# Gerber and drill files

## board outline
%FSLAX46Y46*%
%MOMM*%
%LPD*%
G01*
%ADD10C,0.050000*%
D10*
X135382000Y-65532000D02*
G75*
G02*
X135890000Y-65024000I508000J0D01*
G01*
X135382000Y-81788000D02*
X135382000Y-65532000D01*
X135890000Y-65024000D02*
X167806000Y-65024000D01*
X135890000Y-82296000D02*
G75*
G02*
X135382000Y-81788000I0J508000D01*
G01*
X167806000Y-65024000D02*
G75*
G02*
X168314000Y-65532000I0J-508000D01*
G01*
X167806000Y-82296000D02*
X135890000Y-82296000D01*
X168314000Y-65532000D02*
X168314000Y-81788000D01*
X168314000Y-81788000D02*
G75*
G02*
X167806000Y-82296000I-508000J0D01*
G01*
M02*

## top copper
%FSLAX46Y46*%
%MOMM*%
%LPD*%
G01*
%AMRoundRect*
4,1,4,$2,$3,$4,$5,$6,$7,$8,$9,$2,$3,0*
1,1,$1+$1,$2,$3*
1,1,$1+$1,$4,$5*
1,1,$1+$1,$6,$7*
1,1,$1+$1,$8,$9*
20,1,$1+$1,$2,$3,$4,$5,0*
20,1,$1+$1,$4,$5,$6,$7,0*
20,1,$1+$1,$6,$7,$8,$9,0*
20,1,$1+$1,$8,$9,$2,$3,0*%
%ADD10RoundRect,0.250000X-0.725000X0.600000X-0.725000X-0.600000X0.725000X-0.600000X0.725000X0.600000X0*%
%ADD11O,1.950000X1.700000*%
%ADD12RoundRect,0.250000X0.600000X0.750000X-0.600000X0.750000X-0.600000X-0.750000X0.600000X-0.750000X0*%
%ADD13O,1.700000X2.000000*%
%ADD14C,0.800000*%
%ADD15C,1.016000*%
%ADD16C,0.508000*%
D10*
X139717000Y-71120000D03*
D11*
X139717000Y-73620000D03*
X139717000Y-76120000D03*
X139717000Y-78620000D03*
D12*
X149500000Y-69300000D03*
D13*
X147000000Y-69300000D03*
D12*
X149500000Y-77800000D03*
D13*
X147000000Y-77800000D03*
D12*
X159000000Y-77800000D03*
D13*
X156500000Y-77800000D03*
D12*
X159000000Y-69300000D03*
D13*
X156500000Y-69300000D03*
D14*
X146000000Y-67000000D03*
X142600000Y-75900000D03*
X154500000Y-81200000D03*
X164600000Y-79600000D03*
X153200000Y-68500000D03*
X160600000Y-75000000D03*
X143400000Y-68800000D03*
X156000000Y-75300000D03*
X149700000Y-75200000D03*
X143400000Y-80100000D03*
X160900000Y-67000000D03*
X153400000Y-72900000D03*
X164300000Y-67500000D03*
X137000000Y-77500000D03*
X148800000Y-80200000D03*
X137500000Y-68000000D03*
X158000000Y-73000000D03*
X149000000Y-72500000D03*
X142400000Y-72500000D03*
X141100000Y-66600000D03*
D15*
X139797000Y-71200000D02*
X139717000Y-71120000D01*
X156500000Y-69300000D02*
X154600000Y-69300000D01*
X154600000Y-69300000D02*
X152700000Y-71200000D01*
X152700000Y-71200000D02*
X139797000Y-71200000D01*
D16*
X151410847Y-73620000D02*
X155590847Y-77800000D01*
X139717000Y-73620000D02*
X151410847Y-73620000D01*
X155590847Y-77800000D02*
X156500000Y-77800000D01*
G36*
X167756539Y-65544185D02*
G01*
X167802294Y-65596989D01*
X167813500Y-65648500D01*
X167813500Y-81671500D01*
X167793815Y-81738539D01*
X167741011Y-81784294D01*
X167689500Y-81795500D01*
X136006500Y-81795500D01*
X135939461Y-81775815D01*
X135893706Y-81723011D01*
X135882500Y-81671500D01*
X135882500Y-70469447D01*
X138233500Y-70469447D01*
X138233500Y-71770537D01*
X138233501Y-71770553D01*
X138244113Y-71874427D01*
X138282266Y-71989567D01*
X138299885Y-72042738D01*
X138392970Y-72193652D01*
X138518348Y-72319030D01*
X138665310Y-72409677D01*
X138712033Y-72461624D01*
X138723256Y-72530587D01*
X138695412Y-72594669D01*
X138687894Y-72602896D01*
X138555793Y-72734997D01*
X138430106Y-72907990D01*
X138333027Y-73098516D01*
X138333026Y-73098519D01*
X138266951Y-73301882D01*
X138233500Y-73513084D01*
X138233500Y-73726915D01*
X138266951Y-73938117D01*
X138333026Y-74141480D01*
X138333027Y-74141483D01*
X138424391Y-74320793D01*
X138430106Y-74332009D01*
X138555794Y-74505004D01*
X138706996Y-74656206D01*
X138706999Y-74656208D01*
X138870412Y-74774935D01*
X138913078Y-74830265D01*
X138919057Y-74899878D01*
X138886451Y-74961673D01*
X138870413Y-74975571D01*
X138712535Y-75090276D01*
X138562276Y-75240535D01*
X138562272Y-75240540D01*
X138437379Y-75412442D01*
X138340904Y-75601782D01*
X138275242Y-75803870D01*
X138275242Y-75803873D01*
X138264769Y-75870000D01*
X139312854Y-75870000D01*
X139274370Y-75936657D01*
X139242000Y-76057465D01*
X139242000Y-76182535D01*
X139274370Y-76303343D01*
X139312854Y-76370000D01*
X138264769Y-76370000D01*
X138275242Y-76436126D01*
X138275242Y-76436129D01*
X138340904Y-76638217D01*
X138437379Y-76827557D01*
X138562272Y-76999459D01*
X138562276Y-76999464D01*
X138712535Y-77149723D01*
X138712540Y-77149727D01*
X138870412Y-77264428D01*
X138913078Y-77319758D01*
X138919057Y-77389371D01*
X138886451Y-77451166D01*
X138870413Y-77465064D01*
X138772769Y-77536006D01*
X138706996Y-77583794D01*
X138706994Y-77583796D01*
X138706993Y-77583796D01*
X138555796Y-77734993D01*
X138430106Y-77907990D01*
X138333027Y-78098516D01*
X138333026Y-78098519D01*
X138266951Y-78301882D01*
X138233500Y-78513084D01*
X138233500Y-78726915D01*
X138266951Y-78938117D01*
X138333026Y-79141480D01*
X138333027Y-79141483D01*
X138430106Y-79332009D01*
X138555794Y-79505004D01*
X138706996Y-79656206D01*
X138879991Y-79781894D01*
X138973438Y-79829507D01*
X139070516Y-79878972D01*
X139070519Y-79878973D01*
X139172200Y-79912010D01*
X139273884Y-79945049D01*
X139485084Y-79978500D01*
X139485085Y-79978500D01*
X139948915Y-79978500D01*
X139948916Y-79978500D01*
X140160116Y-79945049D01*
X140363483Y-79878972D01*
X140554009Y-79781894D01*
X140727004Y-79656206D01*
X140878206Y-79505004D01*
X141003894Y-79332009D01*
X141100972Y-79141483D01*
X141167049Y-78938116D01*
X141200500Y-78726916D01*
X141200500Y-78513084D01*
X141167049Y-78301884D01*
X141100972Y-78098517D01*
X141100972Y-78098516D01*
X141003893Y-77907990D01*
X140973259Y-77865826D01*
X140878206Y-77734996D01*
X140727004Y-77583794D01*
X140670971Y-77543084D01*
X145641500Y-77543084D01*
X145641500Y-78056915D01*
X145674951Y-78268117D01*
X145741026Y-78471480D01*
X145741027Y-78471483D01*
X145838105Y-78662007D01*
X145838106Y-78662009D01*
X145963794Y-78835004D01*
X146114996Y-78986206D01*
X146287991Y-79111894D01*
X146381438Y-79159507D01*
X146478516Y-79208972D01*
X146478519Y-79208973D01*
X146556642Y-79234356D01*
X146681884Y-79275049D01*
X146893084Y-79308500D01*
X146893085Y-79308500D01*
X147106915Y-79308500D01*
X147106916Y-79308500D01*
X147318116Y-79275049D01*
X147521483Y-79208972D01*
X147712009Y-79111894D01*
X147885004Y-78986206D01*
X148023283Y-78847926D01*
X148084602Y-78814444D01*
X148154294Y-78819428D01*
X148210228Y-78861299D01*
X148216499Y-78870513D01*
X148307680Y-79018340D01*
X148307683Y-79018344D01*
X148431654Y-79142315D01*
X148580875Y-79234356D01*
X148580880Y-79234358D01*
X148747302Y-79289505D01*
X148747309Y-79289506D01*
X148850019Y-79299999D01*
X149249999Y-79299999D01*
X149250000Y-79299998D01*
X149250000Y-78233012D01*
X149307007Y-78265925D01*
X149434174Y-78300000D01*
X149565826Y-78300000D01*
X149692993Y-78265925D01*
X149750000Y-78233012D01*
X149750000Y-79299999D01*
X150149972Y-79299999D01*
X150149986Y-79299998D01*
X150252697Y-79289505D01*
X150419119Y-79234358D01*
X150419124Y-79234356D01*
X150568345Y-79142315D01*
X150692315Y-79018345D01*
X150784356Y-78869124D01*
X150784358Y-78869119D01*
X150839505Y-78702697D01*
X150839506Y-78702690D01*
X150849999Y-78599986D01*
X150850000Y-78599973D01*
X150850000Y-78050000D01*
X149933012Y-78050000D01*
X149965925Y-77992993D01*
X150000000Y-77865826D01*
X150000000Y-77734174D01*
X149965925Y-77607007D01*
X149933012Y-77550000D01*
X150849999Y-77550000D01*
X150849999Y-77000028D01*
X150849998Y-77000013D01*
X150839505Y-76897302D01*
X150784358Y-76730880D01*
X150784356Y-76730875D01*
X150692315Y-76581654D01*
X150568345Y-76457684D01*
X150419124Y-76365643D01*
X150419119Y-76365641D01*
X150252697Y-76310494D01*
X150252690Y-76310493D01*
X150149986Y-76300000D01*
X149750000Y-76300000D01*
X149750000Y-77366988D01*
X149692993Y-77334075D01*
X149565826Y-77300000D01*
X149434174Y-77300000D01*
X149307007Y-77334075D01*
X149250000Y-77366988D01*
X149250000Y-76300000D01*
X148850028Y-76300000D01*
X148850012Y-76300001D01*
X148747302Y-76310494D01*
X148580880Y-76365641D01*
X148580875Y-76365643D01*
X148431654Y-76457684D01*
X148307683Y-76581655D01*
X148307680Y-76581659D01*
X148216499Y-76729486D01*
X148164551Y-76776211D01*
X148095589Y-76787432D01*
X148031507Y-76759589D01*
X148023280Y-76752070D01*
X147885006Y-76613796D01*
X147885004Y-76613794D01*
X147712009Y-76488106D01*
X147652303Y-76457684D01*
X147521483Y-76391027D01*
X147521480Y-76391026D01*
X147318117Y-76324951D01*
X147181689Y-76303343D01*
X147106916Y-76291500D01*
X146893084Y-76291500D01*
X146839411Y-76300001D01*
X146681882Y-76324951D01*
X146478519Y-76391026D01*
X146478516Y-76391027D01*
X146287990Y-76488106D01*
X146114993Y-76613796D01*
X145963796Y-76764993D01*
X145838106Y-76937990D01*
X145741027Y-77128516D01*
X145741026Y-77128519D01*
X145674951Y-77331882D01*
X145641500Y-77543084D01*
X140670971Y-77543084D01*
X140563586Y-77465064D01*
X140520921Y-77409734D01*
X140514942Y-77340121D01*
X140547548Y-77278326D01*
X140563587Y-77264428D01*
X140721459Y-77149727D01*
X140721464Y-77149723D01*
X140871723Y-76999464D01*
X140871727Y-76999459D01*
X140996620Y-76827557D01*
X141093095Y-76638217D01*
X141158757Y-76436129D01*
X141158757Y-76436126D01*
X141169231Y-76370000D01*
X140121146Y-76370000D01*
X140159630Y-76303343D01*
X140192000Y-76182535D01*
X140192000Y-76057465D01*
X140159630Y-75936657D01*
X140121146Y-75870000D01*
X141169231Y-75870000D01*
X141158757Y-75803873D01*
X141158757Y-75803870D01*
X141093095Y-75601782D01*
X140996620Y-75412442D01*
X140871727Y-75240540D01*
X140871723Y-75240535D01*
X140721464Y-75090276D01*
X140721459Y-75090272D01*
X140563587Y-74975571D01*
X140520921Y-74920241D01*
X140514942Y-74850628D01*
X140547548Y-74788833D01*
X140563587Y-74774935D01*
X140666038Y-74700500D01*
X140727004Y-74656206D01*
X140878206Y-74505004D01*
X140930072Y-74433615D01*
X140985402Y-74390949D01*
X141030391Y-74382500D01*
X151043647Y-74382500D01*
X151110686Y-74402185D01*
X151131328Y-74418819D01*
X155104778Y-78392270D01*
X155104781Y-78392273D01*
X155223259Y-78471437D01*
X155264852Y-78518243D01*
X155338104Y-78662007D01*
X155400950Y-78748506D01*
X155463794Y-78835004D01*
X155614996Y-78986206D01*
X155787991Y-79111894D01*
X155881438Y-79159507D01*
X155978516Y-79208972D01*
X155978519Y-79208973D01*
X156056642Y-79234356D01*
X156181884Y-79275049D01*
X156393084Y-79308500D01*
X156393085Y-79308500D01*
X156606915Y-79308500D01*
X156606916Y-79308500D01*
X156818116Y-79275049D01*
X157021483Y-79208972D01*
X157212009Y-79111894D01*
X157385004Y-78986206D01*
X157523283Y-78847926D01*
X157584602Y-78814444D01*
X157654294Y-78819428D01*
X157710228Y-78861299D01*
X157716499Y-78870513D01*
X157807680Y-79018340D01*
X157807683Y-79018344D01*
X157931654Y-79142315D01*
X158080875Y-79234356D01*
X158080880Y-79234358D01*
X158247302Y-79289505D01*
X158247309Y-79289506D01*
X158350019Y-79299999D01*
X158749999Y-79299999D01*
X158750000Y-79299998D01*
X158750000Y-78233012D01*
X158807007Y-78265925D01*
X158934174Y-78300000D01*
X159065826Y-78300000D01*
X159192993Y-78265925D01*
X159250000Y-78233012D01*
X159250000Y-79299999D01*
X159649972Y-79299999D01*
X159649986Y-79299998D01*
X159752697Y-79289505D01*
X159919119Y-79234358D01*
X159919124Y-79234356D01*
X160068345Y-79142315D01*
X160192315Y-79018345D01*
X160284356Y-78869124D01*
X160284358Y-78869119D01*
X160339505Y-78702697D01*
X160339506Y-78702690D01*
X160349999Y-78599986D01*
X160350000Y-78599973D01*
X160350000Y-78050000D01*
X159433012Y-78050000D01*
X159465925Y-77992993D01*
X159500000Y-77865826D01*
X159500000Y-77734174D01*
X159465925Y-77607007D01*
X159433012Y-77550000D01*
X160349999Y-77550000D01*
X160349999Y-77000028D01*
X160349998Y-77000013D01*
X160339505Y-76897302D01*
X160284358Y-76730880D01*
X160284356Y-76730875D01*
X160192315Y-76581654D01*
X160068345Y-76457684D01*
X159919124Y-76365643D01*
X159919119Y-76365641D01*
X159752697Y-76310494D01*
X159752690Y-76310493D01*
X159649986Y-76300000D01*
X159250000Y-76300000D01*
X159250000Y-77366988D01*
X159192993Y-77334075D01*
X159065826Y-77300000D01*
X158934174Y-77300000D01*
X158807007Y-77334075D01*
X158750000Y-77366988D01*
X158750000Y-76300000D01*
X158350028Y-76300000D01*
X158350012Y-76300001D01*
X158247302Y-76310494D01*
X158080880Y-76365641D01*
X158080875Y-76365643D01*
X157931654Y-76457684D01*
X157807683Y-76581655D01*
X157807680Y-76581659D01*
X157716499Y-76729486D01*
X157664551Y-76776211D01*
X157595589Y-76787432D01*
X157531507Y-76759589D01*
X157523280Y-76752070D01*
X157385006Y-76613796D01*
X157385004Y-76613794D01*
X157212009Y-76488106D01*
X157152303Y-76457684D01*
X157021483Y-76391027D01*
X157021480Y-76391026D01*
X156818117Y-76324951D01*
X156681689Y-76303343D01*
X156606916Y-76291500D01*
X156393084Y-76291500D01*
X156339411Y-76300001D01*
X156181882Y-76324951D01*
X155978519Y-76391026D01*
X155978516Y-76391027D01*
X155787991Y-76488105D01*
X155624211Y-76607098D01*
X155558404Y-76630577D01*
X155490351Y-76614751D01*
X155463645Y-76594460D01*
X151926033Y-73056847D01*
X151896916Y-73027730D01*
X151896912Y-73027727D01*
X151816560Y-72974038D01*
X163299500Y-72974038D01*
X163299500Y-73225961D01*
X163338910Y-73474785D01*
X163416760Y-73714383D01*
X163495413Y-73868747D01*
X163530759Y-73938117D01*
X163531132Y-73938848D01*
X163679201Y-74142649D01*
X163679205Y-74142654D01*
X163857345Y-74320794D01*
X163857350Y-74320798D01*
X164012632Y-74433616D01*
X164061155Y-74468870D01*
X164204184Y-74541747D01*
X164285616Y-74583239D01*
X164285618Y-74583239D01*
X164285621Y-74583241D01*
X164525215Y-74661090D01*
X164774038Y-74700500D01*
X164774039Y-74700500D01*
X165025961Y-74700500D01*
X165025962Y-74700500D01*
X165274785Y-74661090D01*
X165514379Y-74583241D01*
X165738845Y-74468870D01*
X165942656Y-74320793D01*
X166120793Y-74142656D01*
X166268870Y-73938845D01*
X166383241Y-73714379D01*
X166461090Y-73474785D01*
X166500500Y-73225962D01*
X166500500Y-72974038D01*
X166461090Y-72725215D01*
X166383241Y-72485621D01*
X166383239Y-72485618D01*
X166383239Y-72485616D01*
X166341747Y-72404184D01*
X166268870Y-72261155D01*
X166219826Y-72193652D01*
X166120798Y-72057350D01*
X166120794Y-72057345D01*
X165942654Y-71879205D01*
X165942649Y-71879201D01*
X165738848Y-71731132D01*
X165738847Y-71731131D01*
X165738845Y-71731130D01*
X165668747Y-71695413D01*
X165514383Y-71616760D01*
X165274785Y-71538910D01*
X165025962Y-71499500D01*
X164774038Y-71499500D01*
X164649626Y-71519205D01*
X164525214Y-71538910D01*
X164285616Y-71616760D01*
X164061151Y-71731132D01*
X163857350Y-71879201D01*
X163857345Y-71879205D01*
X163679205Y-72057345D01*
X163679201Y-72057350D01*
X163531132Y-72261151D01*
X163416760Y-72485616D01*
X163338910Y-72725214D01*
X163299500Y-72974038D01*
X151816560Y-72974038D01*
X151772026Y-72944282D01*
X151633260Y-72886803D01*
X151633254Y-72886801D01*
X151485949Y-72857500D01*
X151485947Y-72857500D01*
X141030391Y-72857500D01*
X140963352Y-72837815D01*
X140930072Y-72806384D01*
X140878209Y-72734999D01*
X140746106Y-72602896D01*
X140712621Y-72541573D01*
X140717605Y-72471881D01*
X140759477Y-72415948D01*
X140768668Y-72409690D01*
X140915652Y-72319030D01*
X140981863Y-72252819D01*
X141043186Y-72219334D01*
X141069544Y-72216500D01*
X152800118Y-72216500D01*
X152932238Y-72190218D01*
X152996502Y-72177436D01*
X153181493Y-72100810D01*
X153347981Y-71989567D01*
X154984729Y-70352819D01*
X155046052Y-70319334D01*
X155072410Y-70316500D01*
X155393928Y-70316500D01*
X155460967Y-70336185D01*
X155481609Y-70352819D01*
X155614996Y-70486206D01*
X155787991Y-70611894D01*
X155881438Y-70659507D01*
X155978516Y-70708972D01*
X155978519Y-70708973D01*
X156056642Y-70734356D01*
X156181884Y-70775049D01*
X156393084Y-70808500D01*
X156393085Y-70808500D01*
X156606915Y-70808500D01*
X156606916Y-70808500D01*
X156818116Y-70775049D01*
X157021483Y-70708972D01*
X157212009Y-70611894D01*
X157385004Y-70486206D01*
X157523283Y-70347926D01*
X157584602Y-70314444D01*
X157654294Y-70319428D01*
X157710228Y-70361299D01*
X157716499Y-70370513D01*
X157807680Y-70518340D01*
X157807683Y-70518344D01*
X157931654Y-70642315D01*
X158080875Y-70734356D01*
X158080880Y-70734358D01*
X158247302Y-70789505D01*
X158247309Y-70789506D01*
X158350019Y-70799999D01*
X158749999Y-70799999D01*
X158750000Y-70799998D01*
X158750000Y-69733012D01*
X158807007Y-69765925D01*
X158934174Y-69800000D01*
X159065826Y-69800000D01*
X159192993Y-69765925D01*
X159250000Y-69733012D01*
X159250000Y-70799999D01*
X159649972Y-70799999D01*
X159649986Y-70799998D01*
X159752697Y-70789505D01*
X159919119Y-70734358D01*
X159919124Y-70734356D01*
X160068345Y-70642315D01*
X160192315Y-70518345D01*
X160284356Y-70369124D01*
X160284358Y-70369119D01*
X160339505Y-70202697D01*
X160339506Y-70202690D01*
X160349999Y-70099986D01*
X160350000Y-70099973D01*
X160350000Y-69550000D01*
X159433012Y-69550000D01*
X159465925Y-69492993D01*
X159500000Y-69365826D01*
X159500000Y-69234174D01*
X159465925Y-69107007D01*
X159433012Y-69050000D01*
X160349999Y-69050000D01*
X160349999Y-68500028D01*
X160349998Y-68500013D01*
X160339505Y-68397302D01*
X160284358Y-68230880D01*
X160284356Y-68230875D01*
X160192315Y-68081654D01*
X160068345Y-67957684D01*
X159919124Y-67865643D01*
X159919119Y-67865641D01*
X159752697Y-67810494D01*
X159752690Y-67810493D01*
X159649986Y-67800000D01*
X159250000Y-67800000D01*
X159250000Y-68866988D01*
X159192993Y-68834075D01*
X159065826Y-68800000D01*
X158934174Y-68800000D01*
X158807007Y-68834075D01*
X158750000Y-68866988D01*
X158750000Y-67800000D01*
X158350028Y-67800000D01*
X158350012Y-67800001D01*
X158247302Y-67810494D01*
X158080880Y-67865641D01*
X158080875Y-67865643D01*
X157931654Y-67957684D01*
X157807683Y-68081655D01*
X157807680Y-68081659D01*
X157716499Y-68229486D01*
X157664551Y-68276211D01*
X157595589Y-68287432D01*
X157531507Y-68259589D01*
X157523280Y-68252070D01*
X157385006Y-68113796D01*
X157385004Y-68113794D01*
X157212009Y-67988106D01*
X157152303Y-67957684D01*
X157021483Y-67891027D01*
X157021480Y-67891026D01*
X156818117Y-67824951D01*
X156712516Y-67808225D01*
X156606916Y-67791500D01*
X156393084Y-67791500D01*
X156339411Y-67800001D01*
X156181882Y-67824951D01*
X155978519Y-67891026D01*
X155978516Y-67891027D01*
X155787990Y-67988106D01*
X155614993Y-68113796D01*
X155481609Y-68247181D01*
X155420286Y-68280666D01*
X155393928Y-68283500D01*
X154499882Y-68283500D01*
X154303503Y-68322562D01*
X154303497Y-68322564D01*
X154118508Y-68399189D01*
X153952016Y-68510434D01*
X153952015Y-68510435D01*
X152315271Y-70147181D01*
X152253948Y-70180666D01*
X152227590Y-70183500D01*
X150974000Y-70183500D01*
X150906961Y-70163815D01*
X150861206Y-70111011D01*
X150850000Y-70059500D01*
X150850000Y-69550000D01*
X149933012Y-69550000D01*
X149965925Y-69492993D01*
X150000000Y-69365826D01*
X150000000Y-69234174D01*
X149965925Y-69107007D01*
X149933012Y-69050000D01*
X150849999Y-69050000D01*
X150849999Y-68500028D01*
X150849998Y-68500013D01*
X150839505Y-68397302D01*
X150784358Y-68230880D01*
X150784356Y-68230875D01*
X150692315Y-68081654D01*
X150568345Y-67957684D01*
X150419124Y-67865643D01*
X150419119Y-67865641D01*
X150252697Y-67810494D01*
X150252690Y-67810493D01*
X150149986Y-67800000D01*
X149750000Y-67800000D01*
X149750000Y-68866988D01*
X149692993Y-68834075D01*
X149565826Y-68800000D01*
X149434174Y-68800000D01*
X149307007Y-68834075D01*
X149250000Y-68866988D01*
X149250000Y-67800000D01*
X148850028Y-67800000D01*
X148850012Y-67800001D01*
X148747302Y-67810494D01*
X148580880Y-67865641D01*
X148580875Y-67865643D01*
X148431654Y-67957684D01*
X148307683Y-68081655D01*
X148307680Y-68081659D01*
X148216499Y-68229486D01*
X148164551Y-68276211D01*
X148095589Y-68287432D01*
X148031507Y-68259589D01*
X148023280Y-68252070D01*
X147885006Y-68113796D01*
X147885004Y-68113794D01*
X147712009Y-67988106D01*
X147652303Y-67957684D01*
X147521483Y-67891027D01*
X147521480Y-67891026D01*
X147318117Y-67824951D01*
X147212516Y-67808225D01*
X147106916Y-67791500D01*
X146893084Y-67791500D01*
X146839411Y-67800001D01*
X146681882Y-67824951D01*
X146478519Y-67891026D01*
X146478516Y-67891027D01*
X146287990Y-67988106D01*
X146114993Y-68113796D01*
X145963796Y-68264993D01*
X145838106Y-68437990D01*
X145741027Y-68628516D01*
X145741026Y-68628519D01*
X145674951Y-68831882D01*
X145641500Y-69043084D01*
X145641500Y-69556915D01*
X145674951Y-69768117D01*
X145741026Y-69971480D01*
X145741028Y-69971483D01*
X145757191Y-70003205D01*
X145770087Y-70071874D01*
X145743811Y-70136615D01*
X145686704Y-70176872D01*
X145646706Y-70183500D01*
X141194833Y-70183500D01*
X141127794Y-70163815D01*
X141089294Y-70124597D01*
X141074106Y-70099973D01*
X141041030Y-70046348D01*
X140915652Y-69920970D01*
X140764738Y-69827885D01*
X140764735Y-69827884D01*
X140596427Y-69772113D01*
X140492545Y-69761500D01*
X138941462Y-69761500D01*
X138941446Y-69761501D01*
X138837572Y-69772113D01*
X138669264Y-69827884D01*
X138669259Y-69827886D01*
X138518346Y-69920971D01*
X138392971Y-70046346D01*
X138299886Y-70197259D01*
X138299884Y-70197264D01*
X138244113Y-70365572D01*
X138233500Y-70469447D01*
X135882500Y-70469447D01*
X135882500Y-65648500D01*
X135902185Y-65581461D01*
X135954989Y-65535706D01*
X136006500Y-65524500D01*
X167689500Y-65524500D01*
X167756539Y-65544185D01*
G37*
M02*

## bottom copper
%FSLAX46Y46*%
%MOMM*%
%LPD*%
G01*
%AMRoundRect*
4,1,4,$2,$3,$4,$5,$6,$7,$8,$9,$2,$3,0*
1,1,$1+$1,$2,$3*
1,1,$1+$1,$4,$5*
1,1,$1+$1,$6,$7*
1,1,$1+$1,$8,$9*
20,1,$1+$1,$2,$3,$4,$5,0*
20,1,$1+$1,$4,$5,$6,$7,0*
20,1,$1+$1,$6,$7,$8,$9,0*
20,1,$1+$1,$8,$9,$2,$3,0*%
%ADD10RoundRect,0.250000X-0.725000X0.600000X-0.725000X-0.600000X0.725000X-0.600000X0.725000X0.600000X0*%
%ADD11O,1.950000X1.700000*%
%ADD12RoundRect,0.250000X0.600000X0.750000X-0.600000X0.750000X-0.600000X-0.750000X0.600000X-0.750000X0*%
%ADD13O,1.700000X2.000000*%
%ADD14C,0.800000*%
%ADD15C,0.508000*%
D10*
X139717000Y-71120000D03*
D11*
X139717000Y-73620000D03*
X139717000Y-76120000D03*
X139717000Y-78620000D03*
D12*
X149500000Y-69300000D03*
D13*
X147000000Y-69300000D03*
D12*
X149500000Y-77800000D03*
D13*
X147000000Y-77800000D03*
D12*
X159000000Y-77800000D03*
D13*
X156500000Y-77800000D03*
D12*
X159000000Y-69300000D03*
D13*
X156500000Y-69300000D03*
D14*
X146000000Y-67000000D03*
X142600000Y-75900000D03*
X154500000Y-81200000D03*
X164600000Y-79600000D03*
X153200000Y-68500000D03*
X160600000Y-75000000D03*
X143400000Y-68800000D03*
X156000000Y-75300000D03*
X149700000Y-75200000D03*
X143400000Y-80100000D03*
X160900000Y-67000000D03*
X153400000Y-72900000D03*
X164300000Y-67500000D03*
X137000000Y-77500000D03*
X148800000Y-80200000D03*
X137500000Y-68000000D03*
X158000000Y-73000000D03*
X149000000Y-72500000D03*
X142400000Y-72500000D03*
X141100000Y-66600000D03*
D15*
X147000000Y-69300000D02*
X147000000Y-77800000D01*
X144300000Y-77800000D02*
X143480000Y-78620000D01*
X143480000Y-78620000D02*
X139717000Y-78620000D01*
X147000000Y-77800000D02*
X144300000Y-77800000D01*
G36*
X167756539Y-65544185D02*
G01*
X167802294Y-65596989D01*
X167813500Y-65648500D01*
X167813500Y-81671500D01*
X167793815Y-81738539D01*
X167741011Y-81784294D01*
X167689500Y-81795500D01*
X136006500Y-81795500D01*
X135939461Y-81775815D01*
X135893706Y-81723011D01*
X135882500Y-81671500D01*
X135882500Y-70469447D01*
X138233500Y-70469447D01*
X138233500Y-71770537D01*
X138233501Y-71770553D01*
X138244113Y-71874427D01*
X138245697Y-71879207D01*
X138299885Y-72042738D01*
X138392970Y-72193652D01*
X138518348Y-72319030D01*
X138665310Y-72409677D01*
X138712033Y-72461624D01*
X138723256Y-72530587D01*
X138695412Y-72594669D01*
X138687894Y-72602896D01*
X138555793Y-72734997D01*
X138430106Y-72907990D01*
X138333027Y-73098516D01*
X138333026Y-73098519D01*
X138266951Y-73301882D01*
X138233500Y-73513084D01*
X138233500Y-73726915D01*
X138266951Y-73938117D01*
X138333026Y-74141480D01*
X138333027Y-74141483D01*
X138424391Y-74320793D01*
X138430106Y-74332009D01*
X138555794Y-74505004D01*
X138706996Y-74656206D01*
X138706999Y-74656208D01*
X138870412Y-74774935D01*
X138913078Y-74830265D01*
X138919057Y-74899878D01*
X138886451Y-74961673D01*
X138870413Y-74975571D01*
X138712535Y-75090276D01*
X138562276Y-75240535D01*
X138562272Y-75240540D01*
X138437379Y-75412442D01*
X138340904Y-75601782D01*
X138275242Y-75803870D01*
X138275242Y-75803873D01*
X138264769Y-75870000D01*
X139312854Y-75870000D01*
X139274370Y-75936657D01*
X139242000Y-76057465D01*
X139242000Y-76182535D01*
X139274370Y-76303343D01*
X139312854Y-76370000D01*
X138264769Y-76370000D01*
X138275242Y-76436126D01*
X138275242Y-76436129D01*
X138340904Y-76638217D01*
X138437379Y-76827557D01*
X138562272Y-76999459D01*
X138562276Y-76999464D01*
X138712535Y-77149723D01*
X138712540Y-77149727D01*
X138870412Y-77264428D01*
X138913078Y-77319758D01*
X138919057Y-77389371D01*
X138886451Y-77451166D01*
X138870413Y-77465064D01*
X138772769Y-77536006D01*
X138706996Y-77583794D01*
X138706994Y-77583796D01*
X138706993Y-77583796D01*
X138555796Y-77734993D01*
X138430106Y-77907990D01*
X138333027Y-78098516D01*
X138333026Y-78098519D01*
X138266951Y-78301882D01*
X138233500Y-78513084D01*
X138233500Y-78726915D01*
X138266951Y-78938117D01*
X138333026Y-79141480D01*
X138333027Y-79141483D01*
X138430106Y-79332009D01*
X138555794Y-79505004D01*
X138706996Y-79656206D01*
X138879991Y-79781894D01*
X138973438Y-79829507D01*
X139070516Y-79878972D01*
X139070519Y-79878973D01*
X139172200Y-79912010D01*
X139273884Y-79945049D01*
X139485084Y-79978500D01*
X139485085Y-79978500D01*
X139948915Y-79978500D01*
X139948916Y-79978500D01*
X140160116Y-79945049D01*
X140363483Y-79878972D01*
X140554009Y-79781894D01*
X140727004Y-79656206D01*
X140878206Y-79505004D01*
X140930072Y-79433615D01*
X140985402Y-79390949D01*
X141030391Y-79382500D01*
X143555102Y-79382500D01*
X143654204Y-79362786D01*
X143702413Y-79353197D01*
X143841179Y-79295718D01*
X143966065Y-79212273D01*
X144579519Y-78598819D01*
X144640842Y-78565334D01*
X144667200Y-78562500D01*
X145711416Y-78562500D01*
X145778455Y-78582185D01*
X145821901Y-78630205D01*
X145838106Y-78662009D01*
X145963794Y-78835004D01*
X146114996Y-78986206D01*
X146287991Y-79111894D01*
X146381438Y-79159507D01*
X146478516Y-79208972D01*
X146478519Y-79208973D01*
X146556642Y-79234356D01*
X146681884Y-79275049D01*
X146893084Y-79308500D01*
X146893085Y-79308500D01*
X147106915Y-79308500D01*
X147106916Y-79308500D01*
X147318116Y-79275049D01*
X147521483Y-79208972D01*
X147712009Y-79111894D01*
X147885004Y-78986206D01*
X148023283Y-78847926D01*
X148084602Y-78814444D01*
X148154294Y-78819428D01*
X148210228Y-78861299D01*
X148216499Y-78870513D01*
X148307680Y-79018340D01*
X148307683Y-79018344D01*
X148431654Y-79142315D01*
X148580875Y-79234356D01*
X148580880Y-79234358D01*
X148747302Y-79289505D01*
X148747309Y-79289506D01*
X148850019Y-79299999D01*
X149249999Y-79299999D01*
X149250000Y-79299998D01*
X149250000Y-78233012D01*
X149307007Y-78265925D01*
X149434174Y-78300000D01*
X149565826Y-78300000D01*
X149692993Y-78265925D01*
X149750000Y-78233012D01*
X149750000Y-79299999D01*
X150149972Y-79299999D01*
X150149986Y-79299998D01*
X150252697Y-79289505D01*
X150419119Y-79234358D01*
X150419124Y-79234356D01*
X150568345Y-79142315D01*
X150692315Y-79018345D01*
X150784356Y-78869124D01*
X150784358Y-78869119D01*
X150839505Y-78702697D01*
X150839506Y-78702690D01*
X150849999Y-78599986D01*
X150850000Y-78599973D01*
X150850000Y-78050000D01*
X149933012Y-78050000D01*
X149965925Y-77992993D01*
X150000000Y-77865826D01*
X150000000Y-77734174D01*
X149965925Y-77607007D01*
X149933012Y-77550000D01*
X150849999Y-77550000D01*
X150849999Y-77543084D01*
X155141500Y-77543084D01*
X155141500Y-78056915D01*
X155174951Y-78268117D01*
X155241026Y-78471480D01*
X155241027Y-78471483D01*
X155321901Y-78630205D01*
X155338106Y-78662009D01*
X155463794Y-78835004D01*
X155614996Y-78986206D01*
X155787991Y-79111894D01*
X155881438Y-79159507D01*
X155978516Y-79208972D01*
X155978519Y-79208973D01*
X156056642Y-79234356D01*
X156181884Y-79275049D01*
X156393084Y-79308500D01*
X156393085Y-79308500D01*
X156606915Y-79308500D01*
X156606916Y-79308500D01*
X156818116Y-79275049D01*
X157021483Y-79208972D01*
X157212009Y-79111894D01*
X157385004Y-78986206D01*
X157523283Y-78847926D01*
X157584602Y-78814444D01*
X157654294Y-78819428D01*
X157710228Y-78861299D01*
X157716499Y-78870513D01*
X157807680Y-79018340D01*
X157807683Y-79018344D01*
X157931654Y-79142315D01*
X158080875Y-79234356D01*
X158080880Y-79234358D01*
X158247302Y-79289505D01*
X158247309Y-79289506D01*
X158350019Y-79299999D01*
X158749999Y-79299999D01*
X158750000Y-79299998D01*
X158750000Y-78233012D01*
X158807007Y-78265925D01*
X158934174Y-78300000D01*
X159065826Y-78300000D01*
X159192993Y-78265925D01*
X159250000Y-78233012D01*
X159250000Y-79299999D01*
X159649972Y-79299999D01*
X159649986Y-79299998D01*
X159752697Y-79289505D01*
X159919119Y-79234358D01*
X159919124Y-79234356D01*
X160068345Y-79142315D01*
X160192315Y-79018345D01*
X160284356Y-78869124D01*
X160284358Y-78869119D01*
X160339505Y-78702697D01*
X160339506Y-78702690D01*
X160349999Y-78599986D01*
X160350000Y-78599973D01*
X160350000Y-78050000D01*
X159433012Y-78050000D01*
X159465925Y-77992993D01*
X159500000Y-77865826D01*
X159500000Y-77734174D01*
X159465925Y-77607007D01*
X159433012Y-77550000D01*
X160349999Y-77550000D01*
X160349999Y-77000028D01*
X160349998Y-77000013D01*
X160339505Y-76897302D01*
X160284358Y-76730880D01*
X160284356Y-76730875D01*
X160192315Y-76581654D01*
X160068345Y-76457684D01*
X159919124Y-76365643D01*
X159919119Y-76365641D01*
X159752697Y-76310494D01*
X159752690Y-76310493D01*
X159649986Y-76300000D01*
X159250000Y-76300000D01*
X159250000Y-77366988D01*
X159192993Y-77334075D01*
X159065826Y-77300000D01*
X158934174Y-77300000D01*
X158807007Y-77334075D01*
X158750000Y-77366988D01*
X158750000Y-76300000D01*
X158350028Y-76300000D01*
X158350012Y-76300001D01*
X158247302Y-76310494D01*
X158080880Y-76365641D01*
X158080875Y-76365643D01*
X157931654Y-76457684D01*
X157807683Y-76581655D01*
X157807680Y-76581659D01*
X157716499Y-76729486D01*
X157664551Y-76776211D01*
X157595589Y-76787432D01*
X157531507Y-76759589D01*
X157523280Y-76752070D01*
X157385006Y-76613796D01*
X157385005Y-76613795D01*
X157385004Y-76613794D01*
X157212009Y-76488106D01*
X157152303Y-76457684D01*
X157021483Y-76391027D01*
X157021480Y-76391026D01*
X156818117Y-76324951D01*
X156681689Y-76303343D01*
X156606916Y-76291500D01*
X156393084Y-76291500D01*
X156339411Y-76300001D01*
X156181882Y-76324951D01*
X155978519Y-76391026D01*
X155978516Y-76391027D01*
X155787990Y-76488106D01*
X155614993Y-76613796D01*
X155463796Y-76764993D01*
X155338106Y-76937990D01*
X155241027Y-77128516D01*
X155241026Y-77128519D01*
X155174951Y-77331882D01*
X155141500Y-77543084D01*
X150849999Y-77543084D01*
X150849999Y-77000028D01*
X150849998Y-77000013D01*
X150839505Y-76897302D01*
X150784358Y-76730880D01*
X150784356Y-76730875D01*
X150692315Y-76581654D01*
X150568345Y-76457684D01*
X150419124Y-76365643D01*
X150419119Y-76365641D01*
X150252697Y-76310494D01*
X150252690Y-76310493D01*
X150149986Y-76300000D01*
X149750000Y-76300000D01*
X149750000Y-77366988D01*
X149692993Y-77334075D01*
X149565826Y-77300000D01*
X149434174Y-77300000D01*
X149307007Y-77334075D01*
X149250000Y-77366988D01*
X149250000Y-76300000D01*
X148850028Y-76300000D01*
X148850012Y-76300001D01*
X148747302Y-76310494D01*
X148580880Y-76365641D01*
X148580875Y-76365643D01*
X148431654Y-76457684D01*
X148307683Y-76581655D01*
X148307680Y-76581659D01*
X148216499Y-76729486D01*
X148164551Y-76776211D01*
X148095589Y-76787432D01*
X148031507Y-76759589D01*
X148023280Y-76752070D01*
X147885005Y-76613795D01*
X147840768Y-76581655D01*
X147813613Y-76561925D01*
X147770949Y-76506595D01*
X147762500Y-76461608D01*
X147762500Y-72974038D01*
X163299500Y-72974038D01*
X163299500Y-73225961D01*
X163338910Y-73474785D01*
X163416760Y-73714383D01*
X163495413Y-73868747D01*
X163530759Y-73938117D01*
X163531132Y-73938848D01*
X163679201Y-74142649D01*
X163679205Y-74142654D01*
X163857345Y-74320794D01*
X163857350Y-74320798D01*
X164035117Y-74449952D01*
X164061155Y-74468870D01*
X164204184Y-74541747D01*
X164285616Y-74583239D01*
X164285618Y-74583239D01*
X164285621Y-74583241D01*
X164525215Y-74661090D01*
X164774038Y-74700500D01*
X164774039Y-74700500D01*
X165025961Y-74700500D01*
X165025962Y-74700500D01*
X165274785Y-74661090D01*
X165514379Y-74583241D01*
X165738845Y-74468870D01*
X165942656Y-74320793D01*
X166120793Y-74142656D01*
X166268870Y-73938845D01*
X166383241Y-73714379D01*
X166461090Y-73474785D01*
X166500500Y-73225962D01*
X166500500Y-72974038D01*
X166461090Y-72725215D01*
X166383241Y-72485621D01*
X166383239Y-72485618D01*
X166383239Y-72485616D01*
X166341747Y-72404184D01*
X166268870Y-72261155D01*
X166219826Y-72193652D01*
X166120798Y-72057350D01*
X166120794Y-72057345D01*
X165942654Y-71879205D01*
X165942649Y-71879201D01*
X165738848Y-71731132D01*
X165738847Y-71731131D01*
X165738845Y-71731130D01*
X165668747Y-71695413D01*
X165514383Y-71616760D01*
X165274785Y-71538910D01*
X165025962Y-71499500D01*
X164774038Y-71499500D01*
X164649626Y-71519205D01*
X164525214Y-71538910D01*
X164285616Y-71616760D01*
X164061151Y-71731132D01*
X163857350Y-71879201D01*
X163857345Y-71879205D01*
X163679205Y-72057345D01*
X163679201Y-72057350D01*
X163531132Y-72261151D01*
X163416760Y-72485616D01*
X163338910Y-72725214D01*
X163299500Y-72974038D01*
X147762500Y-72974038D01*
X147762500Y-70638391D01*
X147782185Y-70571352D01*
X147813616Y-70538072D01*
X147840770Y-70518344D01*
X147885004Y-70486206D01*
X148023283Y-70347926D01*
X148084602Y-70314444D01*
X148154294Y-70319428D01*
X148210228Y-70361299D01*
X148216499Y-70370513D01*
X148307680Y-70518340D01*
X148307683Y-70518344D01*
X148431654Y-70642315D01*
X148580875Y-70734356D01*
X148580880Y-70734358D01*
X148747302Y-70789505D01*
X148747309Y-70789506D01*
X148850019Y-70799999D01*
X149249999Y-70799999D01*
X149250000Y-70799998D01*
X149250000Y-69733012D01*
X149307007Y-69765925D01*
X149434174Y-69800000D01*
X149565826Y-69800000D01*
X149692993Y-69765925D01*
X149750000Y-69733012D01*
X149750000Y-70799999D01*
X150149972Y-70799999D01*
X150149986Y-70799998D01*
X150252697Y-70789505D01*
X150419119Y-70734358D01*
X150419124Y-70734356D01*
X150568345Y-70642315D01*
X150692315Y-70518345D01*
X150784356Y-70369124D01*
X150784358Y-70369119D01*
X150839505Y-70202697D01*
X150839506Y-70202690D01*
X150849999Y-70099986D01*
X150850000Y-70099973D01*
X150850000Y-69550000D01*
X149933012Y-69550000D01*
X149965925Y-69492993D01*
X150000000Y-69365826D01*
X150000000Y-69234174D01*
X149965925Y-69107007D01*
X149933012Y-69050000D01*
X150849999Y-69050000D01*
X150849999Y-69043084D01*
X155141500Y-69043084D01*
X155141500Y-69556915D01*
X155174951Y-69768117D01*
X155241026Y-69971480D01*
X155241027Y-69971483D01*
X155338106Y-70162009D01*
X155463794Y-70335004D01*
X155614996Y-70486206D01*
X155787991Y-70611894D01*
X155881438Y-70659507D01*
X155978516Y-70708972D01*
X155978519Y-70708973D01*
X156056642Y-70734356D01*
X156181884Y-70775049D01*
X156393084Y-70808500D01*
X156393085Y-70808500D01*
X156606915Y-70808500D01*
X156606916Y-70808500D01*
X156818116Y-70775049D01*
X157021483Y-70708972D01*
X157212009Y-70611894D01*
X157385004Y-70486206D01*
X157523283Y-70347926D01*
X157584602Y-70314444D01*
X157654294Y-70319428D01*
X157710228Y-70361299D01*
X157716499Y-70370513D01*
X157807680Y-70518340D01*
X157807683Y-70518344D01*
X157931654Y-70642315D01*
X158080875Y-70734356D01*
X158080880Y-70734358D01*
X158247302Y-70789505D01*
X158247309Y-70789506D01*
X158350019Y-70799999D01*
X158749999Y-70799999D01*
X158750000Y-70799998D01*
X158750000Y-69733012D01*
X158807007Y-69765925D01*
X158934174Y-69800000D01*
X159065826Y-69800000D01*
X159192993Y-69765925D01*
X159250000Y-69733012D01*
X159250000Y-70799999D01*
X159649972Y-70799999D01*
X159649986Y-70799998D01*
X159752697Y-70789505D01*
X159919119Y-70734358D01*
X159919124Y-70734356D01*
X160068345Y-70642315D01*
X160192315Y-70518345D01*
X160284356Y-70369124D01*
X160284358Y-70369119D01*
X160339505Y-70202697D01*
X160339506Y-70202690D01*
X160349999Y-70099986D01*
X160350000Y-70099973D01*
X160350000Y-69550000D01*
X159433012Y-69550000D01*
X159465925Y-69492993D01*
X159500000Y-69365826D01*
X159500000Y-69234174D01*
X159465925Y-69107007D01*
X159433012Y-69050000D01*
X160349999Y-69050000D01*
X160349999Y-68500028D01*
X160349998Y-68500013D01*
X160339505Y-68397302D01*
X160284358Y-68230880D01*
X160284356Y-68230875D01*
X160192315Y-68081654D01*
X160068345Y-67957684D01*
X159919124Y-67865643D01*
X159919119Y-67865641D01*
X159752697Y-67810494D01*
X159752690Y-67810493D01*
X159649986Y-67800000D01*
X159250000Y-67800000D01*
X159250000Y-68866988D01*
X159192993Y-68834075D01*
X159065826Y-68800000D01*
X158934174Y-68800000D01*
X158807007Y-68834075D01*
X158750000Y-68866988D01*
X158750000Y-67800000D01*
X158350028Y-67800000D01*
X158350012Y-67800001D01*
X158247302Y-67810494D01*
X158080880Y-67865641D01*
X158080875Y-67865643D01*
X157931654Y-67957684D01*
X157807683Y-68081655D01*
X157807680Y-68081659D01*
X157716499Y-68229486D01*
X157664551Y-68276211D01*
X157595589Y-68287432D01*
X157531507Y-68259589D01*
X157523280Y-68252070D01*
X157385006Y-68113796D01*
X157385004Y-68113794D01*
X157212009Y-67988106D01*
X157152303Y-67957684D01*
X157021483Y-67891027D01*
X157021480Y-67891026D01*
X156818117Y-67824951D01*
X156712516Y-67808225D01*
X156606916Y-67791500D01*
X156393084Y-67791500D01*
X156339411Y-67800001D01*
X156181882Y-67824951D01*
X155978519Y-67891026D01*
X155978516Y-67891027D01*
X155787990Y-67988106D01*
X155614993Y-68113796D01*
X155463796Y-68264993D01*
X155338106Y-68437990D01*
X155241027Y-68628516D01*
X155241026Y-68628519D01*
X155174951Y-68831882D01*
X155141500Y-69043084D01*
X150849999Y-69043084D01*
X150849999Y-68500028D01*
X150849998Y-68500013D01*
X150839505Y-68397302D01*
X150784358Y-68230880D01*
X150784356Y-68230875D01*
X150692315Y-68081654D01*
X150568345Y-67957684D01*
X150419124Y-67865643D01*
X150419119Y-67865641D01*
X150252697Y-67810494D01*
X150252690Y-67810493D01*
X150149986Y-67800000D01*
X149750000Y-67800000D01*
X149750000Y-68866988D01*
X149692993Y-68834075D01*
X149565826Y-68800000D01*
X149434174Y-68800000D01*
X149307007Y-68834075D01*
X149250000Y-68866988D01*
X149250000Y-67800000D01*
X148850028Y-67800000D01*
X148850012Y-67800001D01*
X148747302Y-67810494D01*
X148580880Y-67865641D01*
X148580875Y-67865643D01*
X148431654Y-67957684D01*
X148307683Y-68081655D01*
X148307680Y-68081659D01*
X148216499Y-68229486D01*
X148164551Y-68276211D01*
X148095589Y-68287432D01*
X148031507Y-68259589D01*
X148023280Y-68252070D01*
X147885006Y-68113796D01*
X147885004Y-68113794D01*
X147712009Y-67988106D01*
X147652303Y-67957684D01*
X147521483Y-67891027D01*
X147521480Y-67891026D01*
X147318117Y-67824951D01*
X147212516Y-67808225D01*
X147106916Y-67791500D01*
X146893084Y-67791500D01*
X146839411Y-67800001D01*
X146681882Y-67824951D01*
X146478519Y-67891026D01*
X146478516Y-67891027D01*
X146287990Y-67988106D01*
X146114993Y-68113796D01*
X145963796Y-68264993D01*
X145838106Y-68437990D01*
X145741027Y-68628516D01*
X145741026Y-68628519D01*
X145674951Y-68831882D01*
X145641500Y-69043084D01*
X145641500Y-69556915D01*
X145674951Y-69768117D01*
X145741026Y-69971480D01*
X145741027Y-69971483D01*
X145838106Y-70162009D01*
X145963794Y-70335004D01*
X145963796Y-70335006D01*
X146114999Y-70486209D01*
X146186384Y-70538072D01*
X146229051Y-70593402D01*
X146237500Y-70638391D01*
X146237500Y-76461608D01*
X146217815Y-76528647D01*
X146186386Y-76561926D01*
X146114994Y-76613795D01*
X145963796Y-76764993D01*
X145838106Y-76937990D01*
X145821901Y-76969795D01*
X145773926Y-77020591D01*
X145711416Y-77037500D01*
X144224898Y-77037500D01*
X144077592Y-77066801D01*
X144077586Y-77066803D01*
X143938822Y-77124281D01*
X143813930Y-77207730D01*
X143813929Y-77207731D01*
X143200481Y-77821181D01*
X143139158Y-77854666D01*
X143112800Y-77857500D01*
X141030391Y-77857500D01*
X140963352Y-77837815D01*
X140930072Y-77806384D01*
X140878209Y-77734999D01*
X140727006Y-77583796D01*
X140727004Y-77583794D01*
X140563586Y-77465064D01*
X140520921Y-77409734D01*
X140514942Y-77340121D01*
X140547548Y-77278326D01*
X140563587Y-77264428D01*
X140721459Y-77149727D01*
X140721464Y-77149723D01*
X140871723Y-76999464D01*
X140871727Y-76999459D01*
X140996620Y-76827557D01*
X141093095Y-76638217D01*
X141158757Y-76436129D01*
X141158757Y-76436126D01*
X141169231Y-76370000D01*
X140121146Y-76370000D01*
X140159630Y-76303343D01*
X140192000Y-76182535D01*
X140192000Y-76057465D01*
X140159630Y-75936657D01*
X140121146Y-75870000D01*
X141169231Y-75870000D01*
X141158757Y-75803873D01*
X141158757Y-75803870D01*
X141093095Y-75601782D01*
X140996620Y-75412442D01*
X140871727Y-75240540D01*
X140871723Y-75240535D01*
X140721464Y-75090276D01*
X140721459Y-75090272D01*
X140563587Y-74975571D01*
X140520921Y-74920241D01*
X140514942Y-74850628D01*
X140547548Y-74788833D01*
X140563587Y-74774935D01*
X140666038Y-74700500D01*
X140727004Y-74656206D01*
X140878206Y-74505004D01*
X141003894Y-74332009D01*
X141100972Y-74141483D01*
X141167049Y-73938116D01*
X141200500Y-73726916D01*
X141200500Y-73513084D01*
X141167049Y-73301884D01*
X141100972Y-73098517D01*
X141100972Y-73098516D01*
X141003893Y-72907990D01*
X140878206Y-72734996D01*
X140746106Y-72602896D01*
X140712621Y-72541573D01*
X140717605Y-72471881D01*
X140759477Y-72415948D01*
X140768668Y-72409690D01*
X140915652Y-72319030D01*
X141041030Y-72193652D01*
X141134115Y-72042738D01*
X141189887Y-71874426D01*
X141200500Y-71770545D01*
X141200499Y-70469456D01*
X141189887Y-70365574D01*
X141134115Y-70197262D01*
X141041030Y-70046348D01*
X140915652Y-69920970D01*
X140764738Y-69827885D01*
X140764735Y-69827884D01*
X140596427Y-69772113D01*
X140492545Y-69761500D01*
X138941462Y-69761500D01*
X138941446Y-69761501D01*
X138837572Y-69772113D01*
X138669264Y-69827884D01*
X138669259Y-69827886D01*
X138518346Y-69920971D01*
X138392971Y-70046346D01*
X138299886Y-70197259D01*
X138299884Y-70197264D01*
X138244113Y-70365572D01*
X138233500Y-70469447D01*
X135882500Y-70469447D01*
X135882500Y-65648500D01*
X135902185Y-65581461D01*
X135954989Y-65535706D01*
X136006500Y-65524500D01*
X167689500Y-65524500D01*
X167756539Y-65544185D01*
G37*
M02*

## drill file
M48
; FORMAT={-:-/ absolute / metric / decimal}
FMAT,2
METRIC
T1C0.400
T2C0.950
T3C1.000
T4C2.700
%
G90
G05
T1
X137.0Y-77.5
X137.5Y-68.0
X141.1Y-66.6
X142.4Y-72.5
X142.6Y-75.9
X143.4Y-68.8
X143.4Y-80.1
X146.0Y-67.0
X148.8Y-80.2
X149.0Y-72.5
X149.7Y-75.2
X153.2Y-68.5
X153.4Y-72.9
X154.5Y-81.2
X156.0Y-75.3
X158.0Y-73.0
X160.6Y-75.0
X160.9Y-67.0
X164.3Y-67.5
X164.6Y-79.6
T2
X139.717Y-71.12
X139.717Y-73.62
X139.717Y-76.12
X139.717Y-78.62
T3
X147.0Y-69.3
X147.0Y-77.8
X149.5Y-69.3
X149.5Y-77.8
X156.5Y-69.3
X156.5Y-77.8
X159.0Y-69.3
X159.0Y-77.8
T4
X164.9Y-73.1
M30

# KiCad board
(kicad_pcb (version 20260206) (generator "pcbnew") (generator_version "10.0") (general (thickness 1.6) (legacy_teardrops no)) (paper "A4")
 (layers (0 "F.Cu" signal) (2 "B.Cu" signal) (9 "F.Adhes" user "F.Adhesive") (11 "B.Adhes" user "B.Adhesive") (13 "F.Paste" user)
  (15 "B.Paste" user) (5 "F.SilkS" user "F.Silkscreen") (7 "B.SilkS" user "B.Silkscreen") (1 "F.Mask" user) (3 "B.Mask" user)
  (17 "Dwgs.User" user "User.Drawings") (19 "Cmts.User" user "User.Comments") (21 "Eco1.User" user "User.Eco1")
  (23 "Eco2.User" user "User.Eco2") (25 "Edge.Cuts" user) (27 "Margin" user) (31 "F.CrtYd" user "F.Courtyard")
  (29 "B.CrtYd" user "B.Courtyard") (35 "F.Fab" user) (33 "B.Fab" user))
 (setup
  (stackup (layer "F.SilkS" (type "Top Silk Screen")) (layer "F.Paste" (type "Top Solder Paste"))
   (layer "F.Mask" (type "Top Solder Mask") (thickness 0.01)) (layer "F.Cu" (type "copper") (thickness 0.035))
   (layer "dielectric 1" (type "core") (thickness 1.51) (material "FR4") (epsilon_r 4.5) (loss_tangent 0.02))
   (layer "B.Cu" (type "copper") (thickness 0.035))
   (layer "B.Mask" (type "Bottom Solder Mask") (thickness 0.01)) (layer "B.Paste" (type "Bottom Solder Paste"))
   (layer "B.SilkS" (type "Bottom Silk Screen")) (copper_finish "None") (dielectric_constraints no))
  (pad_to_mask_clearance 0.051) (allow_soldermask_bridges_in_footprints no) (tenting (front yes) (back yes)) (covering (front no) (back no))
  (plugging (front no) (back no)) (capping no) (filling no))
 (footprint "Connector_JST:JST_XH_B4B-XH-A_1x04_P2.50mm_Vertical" (layer "F.Cu") (at 139.717 71.12 -90)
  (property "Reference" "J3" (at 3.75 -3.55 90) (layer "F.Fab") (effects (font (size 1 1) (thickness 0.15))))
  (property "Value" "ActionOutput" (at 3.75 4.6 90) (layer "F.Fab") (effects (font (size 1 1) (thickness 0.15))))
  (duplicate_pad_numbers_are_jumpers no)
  (pad "1" thru_hole roundrect (at 0 0 270) (size 1.7 1.95) (drill 0.95) (layers "*.Cu" "*.Mask") (remove_unused_layers no)
   (roundrect_rratio 0.147059) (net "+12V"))
  (pad "2" thru_hole oval (at 2.5 0 270) (size 1.7 1.95) (drill 0.95) (layers "*.Cu" "*.Mask") (remove_unused_layers no) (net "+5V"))
  (pad "3" thru_hole oval (at 5 0 270) (size 1.7 1.95) (drill 0.95) (layers "*.Cu" "*.Mask") (remove_unused_layers no) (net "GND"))
  (pad "4" thru_hole oval (at 7.5 0 270) (size 1.7 1.95) (drill 0.95) (layers "*.Cu" "*.Mask") (remove_unused_layers no)
   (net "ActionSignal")))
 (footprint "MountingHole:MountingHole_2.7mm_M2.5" (layer "F.Cu") (at 164.9 73.1)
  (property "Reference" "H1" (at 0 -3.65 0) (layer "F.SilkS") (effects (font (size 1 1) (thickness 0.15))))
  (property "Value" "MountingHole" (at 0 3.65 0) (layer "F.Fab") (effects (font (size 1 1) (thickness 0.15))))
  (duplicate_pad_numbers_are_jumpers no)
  (pad "" np_thru_hole circle (at 0 0) (size 2.7 2.7) (drill 2.7) (layers "*.Cu" "*.Mask")))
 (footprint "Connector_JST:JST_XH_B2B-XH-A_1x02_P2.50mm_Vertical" (layer "F.Cu") (at 149.5 69.3 180)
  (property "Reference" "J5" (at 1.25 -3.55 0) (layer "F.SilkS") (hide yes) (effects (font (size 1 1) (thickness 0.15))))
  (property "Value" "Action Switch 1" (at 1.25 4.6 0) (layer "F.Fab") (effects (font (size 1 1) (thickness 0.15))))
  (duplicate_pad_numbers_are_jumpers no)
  (pad "1" thru_hole roundrect (at 0 0 180) (size 1.7 2) (drill 1) (layers "*.Cu" "*.Mask") (remove_unused_layers no)
   (roundrect_rratio 0.147059) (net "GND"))
  (pad "2" thru_hole oval (at 2.5 0 180) (size 1.7 2) (drill 1) (layers "*.Cu" "*.Mask") (remove_unused_layers no) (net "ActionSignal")))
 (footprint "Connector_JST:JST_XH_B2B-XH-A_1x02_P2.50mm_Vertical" (layer "F.Cu") (at 149.5 77.8 180)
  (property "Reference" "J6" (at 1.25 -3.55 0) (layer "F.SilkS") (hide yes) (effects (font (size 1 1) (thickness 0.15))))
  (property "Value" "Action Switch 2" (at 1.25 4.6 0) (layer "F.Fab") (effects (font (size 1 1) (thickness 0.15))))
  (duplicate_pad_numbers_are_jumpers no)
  (pad "1" thru_hole roundrect (at 0 0 180) (size 1.7 2) (drill 1) (layers "*.Cu" "*.Mask") (remove_unused_layers no)
   (roundrect_rratio 0.147059) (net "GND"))
  (pad "2" thru_hole oval (at 2.5 0 180) (size 1.7 2) (drill 1) (layers "*.Cu" "*.Mask") (remove_unused_layers no) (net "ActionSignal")))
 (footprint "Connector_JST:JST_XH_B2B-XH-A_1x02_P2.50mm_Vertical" (layer "F.Cu") (at 159 77.8 180)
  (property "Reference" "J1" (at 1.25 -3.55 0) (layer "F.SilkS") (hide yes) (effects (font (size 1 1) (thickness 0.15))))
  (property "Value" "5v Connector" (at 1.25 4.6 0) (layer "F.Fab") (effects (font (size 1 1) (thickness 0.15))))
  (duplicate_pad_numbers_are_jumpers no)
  (pad "1" thru_hole roundrect (at 0 0 180) (size 1.7 2) (drill 1) (layers "*.Cu" "*.Mask") (remove_unused_layers no)
   (roundrect_rratio 0.147059) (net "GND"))
  (pad "2" thru_hole oval (at 2.5 0 180) (size 1.7 2) (drill 1) (layers "*.Cu" "*.Mask") (remove_unused_layers no) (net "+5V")))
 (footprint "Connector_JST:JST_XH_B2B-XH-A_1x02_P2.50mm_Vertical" (layer "F.Cu") (at 159 69.3 180)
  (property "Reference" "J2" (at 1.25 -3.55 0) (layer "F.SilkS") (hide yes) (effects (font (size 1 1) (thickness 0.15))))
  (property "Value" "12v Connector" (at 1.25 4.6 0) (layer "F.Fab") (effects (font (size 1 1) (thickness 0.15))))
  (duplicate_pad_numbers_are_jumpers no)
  (pad "1" thru_hole roundrect (at 0 0 180) (size 1.7 2) (drill 1) (layers "*.Cu" "*.Mask") (remove_unused_layers no)
   (roundrect_rratio 0.147059) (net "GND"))
  (pad "2" thru_hole oval (at 2.5 0 180) (size 1.7 2) (drill 1) (layers "*.Cu" "*.Mask") (remove_unused_layers no) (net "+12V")))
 (gr_arc (start 135.382 65.532) (mid 135.53079 65.17279) (end 135.89 65.024) (stroke (width 0.05) (type default)) (layer "Edge.Cuts"))
 (gr_line (start 135.382 81.788) (end 135.382 65.532) (stroke (width 0.05) (type solid)) (layer "Edge.Cuts"))
 (gr_line (start 135.89 65.024) (end 167.806 65.024) (stroke (width 0.05) (type solid)) (layer "Edge.Cuts"))
 (gr_arc (start 135.89 82.296) (mid 135.53079 82.14721) (end 135.382 81.788) (stroke (width 0.05) (type default)) (layer "Edge.Cuts"))
 (gr_arc (start 167.806 65.024) (mid 168.16521 65.17279) (end 168.314 65.532) (stroke (width 0.05) (type default)) (layer "Edge.Cuts"))
 (gr_line (start 167.806 82.296) (end 135.89 82.296) (stroke (width 0.05) (type solid)) (layer "Edge.Cuts"))
 (gr_line (start 168.314 65.532) (end 168.314 81.788) (stroke (width 0.05) (type solid)) (layer "Edge.Cuts"))
 (gr_arc (start 168.314 81.788) (mid 168.16521 82.14721) (end 167.806 82.296) (stroke (width 0.05) (type default)) (layer "Edge.Cuts"))
 (segment (start 139.797 71.2) (end 139.717 71.12) (width 1.016) (layer "F.Cu") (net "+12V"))
 (segment (start 156.5 69.3) (end 154.6 69.3) (width 1.016) (layer "F.Cu") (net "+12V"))
 (segment (start 154.6 69.3) (end 152.7 71.2) (width 1.016) (layer "F.Cu") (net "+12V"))
 (segment (start 152.7 71.2) (end 139.797 71.2) (width 1.016) (layer "F.Cu") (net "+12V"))
 (segment (start 151.410847 73.62) (end 155.590847 77.8) (width 0.508) (layer "F.Cu") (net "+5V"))
 (segment (start 139.717 73.62) (end 151.410847 73.62) (width 0.508) (layer "F.Cu") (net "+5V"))
 (segment (start 155.590847 77.8) (end 156.5 77.8) (width 0.508) (layer "F.Cu") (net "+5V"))
 (via (at 146 67) (size 0.8) (drill 0.4) (layers "F.Cu" "B.Cu") (free yes) (capping no) (covering (front no) (back no))
  (plugging (front no) (back no)) (filling no) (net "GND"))
 (via (at 142.6 75.9) (size 0.8) (drill 0.4) (layers "F.Cu" "B.Cu") (free yes) (capping no) (covering (front no) (back no))
  (plugging (front no) (back no)) (filling no) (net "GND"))
 (via (at 154.5 81.2) (size 0.8) (drill 0.4) (layers "F.Cu" "B.Cu") (free yes) (capping no) (covering (front no) (back no))
  (plugging (front no) (back no)) (filling no) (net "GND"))
 (via (at 164.6 79.6) (size 0.8) (drill 0.4) (layers "F.Cu" "B.Cu") (free yes) (capping no) (covering (front no) (back no))
  (plugging (front no) (back no)) (filling no) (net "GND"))
 (via (at 153.2 68.5) (size 0.8) (drill 0.4) (layers "F.Cu" "B.Cu") (free yes) (capping no) (covering (front no) (back no))
  (plugging (front no) (back no)) (filling no) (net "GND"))
 (via (at 160.6 75) (size 0.8) (drill 0.4) (layers "F.Cu" "B.Cu") (free yes) (capping no) (covering (front no) (back no))
  (plugging (front no) (back no)) (filling no) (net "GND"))
 (via (at 143.4 68.8) (size 0.8) (drill 0.4) (layers "F.Cu" "B.Cu") (free yes) (capping no) (covering (front no) (back no))
  (plugging (front no) (back no)) (filling no) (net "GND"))
 (via (at 156 75.3) (size 0.8) (drill 0.4) (layers "F.Cu" "B.Cu") (free yes) (capping no) (covering (front no) (back no))
  (plugging (front no) (back no)) (filling no) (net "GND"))
 (via (at 149.7 75.2) (size 0.8) (drill 0.4) (layers "F.Cu" "B.Cu") (free yes) (capping no) (covering (front no) (back no))
  (plugging (front no) (back no)) (filling no) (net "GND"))
 (via (at 143.4 80.1) (size 0.8) (drill 0.4) (layers "F.Cu" "B.Cu") (free yes) (capping no) (covering (front no) (back no))
  (plugging (front no) (back no)) (filling no) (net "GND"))
 (via (at 160.9 67) (size 0.8) (drill 0.4) (layers "F.Cu" "B.Cu") (free yes) (capping no) (covering (front no) (back no))
  (plugging (front no) (back no)) (filling no) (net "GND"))
 (via (at 153.4 72.9) (size 0.8) (drill 0.4) (layers "F.Cu" "B.Cu") (free yes) (capping no) (covering (front no) (back no))
  (plugging (front no) (back no)) (filling no) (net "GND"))
 (via (at 164.3 67.5) (size 0.8) (drill 0.4) (layers "F.Cu" "B.Cu") (free yes) (capping no) (covering (front no) (back no))
  (plugging (front no) (back no)) (filling no) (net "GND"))
 (via (at 137 77.5) (size 0.8) (drill 0.4) (layers "F.Cu" "B.Cu") (free yes) (capping no) (covering (front no) (back no))
  (plugging (front no) (back no)) (filling no) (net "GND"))
 (via (at 148.8 80.2) (size 0.8) (drill 0.4) (layers "F.Cu" "B.Cu") (free yes) (capping no) (covering (front no) (back no))
  (plugging (front no) (back no)) (filling no) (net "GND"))
 (via (at 137.5 68) (size 0.8) (drill 0.4) (layers "F.Cu" "B.Cu") (free yes) (capping no) (covering (front no) (back no))
  (plugging (front no) (back no)) (filling no) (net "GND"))
 (via (at 158 73) (size 0.8) (drill 0.4) (layers "F.Cu" "B.Cu") (free yes) (capping no) (covering (front no) (back no))
  (plugging (front no) (back no)) (filling no) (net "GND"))
 (via (at 149 72.5) (size 0.8) (drill 0.4) (layers "F.Cu" "B.Cu") (free yes) (capping no) (covering (front no) (back no))
  (plugging (front no) (back no)) (filling no) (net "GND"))
 (via (at 142.4 72.5) (size 0.8) (drill 0.4) (layers "F.Cu" "B.Cu") (free yes) (capping no) (covering (front no) (back no))
  (plugging (front no) (back no)) (filling no) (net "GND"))
 (via (at 141.1 66.6) (size 0.8) (drill 0.4) (layers "F.Cu" "B.Cu") (free yes) (capping no) (covering (front no) (back no))
  (plugging (front no) (back no)) (filling no) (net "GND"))
 (segment (start 147 69.3) (end 147 77.8) (width 0.508) (layer "B.Cu") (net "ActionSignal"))
 (segment (start 144.3 77.8) (end 143.48 78.62) (width 0.508) (layer "B.Cu") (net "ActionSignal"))
 (segment (start 143.48 78.62) (end 139.717 78.62) (width 0.508) (layer "B.Cu") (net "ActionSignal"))
 (segment (start 147 77.8) (end 144.3 77.8) (width 0.508) (layer "B.Cu") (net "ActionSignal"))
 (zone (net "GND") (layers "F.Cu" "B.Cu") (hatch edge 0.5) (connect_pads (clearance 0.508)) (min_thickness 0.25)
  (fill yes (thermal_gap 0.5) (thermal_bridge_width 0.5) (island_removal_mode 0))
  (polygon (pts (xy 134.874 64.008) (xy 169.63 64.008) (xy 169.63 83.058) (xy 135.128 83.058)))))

